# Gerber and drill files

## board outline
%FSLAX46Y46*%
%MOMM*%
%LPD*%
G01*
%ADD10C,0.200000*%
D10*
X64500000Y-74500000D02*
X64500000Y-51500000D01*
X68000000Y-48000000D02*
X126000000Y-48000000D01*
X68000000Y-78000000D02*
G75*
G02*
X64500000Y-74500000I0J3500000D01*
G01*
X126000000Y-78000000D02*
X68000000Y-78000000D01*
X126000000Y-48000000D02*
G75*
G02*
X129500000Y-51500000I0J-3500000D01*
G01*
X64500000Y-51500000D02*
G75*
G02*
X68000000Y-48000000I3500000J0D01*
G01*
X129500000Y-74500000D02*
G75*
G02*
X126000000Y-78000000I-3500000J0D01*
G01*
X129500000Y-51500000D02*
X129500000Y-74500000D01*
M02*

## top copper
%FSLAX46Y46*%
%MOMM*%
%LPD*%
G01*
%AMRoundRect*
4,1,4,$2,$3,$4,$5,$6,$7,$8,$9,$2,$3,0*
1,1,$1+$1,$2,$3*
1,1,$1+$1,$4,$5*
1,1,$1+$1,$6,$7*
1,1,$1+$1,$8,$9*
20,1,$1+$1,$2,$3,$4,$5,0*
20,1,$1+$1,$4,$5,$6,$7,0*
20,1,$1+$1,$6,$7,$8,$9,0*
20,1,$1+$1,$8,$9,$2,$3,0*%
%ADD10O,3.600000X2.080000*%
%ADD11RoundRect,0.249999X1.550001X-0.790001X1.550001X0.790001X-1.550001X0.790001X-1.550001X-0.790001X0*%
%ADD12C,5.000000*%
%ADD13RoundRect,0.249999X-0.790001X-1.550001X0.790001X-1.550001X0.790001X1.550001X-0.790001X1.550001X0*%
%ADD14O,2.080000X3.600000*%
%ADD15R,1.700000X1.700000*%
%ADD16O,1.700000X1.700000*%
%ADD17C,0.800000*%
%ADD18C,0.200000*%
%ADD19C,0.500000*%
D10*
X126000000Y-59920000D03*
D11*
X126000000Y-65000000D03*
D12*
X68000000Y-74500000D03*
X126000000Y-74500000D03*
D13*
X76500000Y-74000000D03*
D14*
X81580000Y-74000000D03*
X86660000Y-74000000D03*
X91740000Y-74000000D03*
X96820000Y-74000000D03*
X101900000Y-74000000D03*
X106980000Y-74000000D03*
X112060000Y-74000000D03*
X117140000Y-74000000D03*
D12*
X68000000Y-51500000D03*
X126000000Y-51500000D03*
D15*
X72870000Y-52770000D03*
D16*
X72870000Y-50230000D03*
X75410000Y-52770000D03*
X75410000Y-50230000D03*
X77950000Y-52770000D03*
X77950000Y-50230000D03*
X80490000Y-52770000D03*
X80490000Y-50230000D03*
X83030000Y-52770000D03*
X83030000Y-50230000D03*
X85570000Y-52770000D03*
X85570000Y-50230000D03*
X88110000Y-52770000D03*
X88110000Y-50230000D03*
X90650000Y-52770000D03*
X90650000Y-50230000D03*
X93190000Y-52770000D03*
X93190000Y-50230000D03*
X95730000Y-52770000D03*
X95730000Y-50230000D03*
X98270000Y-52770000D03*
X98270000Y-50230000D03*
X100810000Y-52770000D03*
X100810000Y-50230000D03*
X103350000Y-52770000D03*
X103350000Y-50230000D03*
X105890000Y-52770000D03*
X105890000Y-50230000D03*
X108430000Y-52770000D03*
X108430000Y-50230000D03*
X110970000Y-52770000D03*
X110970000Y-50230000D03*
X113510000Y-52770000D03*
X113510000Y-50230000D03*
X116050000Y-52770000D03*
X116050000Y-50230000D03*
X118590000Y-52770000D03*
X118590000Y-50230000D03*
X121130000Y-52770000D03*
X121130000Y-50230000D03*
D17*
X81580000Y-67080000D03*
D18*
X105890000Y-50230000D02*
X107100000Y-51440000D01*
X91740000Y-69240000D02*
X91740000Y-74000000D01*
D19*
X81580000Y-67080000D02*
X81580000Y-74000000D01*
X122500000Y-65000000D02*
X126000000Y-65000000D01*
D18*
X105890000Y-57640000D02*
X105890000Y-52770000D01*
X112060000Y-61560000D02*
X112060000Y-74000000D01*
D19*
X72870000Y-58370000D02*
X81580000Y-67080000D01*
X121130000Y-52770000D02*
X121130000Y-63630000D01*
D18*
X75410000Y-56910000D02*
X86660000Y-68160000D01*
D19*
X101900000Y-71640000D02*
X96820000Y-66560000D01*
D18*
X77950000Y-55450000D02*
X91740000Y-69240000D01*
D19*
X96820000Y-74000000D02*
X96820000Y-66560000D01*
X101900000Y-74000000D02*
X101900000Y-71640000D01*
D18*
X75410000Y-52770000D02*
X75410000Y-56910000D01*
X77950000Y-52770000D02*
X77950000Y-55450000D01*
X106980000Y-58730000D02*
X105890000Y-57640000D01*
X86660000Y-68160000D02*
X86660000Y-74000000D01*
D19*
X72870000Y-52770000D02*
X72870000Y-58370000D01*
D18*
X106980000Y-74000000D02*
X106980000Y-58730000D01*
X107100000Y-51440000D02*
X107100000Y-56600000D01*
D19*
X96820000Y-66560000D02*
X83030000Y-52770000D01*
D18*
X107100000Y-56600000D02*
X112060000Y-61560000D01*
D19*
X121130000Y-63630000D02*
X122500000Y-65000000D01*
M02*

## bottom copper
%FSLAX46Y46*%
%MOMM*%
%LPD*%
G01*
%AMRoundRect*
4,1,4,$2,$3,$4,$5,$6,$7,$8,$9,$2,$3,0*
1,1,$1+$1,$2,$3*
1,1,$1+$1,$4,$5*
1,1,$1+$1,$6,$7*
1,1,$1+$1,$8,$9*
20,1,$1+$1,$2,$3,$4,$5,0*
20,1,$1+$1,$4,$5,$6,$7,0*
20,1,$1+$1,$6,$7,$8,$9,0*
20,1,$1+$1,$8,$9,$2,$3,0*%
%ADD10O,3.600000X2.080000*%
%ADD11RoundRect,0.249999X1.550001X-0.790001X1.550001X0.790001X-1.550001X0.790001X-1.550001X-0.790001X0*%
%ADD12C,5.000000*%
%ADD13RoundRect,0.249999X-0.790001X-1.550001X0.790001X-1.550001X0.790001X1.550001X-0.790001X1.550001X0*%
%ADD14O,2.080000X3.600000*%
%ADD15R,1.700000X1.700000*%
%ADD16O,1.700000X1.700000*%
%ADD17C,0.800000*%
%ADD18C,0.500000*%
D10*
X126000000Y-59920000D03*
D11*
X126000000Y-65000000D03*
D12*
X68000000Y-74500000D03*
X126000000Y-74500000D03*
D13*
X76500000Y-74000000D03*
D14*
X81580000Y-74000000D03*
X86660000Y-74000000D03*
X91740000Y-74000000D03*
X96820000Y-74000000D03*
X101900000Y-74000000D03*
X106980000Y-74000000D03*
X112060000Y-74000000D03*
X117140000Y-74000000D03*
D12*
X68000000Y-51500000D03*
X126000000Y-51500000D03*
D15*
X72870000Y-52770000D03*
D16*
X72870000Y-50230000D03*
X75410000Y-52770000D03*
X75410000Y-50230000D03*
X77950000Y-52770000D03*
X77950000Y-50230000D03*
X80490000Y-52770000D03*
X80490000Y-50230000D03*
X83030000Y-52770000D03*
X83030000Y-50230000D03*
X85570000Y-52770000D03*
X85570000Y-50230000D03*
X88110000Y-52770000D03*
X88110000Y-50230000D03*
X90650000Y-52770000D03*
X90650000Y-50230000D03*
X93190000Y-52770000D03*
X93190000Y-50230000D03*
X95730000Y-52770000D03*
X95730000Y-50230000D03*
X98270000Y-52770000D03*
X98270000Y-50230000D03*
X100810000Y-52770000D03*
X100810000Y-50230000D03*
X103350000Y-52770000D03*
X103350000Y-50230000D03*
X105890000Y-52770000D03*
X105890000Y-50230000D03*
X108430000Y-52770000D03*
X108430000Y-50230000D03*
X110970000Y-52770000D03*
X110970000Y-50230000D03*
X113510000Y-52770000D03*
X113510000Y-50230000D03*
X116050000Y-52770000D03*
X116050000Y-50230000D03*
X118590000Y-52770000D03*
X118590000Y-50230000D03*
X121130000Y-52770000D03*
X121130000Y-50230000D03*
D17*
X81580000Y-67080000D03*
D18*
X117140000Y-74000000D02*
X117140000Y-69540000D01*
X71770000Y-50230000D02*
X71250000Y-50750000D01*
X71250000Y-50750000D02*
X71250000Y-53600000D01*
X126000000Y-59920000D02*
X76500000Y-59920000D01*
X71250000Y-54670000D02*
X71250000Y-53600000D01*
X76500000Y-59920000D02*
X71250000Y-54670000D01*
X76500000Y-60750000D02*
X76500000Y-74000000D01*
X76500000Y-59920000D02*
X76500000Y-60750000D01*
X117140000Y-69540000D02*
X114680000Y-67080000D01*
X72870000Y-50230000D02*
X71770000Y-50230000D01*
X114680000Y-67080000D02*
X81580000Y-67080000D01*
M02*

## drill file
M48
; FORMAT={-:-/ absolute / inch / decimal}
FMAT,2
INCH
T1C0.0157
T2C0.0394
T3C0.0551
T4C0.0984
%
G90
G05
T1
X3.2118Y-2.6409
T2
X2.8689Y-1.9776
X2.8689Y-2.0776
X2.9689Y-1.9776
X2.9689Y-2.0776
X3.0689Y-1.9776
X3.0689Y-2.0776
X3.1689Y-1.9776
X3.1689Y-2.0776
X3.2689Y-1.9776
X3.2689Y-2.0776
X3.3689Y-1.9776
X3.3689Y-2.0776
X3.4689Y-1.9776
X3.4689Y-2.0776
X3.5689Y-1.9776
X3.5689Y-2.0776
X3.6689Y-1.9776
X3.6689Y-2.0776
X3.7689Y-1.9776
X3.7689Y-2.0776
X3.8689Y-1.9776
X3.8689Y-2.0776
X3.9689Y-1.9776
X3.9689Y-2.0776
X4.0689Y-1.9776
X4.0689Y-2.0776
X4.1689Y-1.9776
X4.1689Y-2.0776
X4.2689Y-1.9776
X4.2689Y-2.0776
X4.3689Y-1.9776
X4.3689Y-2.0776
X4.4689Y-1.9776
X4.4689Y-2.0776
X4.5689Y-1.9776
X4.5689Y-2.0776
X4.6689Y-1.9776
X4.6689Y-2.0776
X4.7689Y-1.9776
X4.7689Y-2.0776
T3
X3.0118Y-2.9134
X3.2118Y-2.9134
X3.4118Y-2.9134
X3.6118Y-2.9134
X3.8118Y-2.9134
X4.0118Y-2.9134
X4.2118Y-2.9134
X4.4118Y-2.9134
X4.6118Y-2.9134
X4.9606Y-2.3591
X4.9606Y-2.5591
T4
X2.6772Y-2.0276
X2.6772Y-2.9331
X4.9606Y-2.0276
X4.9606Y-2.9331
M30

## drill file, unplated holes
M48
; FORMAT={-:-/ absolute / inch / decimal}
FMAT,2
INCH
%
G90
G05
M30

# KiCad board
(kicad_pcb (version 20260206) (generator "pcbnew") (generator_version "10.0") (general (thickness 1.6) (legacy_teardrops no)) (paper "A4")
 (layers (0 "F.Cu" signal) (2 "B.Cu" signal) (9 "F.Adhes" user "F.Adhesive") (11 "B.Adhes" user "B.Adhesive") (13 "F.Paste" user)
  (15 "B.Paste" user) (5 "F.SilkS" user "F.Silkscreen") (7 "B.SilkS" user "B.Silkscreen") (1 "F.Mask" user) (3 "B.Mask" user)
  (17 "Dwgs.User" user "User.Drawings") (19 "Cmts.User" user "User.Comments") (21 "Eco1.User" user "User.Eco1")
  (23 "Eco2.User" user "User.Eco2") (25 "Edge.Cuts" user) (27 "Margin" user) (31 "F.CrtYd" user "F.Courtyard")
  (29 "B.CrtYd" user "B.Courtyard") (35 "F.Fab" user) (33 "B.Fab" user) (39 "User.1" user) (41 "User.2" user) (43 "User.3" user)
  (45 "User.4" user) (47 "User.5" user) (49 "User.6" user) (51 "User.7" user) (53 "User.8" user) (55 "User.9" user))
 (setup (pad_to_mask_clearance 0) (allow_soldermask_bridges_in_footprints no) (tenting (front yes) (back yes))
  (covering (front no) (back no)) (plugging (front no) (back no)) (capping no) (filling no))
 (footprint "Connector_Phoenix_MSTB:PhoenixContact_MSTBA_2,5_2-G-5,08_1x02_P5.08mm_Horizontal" (layer "F.Cu") (at 126 65 90)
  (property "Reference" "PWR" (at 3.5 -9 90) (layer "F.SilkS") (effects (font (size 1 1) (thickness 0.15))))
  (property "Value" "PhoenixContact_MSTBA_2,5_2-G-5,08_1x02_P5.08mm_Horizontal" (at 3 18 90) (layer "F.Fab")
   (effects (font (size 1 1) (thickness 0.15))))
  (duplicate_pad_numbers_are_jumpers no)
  (pad "1" thru_hole roundrect (at 0 0 90) (size 2.08 3.6) (drill 1.4) (layers "*.Cu" "*.Mask") (remove_unused_layers no)
   (roundrect_rratio 0.120192))
  (pad "2" thru_hole oval (at 5.08 0 90) (size 2.08 3.6) (drill 1.4) (layers "*.Cu" "*.Mask") (remove_unused_layers no)))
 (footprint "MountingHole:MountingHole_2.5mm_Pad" (layer "F.Cu") (at 68 74.5)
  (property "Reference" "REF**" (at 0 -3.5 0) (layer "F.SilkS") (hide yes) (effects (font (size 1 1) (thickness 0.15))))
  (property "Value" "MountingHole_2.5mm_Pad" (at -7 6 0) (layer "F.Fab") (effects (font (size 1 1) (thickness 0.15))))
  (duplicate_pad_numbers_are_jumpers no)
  (pad "1" thru_hole circle (at 0 0) (size 5 5) (drill 2.5) (layers "*.Cu" "*.Mask") (remove_unused_layers no)))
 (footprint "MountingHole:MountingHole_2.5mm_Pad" (layer "F.Cu") (at 126 74.5)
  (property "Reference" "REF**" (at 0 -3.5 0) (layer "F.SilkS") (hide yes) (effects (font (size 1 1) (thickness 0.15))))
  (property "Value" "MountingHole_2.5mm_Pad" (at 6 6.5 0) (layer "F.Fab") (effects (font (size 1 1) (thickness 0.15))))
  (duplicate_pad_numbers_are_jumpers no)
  (pad "1" thru_hole circle (at 0 0) (size 5 5) (drill 2.5) (layers "*.Cu" "*.Mask") (remove_unused_layers no)))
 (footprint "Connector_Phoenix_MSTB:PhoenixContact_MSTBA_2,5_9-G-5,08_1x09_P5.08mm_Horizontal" (layer "F.Cu") (at 76.5 74)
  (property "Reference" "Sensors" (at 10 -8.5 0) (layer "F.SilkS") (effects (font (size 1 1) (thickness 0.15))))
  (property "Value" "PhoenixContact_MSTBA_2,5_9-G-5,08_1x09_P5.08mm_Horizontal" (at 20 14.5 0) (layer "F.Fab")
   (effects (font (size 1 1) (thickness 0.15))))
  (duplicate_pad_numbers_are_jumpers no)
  (pad "1" thru_hole roundrect (at 0 0) (size 2.08 3.6) (drill 1.4) (layers "*.Cu" "*.Mask") (remove_unused_layers no)
   (roundrect_rratio 0.120192))
  (pad "2" thru_hole oval (at 5.08 0) (size 2.08 3.6) (drill 1.4) (layers "*.Cu" "*.Mask") (remove_unused_layers no))
  (pad "3" thru_hole oval (at 10.16 0) (size 2.08 3.6) (drill 1.4) (layers "*.Cu" "*.Mask") (remove_unused_layers no))
  (pad "4" thru_hole oval (at 15.24 0) (size 2.08 3.6) (drill 1.4) (layers "*.Cu" "*.Mask") (remove_unused_layers no))
  (pad "5" thru_hole oval (at 20.32 0) (size 2.08 3.6) (drill 1.4) (layers "*.Cu" "*.Mask") (remove_unused_layers no))
  (pad "6" thru_hole oval (at 25.4 0) (size 2.08 3.6) (drill 1.4) (layers "*.Cu" "*.Mask") (remove_unused_layers no))
  (pad "7" thru_hole oval (at 30.48 0) (size 2.08 3.6) (drill 1.4) (layers "*.Cu" "*.Mask") (remove_unused_layers no))
  (pad "8" thru_hole oval (at 35.56 0) (size 2.08 3.6) (drill 1.4) (layers "*.Cu" "*.Mask") (remove_unused_layers no))
  (pad "9" thru_hole oval (at 40.64 0) (size 2.08 3.6) (drill 1.4) (layers "*.Cu" "*.Mask") (remove_unused_layers no)))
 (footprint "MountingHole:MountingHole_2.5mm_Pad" (layer "F.Cu") (at 68 51.5)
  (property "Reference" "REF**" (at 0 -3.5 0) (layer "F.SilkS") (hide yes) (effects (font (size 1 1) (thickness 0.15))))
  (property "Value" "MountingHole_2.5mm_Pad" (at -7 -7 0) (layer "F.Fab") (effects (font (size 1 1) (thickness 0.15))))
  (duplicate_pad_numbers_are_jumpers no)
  (pad "1" thru_hole circle (at 0 0) (size 5 5) (drill 2.5) (layers "*.Cu" "*.Mask") (remove_unused_layers no)))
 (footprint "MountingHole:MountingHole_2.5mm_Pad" (layer "F.Cu") (at 126 51.5)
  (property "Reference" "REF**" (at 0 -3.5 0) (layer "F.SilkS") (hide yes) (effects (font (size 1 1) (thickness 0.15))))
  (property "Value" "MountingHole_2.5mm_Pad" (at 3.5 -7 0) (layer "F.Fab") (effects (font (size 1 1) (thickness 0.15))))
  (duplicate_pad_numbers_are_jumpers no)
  (pad "1" thru_hole circle (at 0 0) (size 5 5) (drill 2.5) (layers "*.Cu" "*.Mask") (remove_unused_layers no)))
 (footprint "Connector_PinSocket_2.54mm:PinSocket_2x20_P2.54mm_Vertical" (layer "B.Cu") (at 121.16 50.2 90)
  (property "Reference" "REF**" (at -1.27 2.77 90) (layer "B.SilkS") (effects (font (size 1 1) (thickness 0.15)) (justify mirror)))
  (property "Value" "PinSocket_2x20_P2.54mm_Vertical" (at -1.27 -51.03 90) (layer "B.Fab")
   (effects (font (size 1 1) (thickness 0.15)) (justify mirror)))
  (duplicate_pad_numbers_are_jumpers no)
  (pad "1" thru_hole rect (at 0 0 90) (size 1.7 1.7) (drill 1) (layers "*.Cu" "*.Mask") (remove_unused_layers no))
  (pad "2" thru_hole circle (at -2.54 0 90) (size 1.7 1.7) (drill 1) (layers "*.Cu" "*.Mask") (remove_unused_layers no))
  (pad "3" thru_hole circle (at 0 -2.54 90) (size 1.7 1.7) (drill 1) (layers "*.Cu" "*.Mask") (remove_unused_layers no))
  (pad "4" thru_hole circle (at -2.54 -2.54 90) (size 1.7 1.7) (drill 1) (layers "*.Cu" "*.Mask") (remove_unused_layers no))
  (pad "5" thru_hole circle (at 0 -5.08 90) (size 1.7 1.7) (drill 1) (layers "*.Cu" "*.Mask") (remove_unused_layers no))
  (pad "6" thru_hole circle (at -2.54 -5.08 90) (size 1.7 1.7) (drill 1) (layers "*.Cu" "*.Mask") (remove_unused_layers no))
  (pad "7" thru_hole circle (at 0 -7.62 90) (size 1.7 1.7) (drill 1) (layers "*.Cu" "*.Mask") (remove_unused_layers no))
  (pad "8" thru_hole circle (at -2.54 -7.62 90) (size 1.7 1.7) (drill 1) (layers "*.Cu" "*.Mask") (remove_unused_layers no))
  (pad "9" thru_hole circle (at 0 -10.16 90) (size 1.7 1.7) (drill 1) (layers "*.Cu" "*.Mask") (remove_unused_layers no))
  (pad "10" thru_hole circle (at -2.54 -10.16 90) (size 1.7 1.7) (drill 1) (layers "*.Cu" "*.Mask") (remove_unused_layers no))
  (pad "11" thru_hole circle (at 0 -12.7 90) (size 1.7 1.7) (drill 1) (layers "*.Cu" "*.Mask") (remove_unused_layers no))
  (pad "12" thru_hole circle (at -2.54 -12.7 90) (size 1.7 1.7) (drill 1) (layers "*.Cu" "*.Mask") (remove_unused_layers no))
  (pad "13" thru_hole circle (at 0 -15.24 90) (size 1.7 1.7) (drill 1) (layers "*.Cu" "*.Mask") (remove_unused_layers no))
  (pad "14" thru_hole circle (at -2.54 -15.24 90) (size 1.7 1.7) (drill 1) (layers "*.Cu" "*.Mask") (remove_unused_layers no))
  (pad "15" thru_hole circle (at 0 -17.78 90) (size 1.7 1.7) (drill 1) (layers "*.Cu" "*.Mask") (remove_unused_layers no))
  (pad "16" thru_hole circle (at -2.54 -17.78 90) (size 1.7 1.7) (drill 1) (layers "*.Cu" "*.Mask") (remove_unused_layers no))
  (pad "17" thru_hole circle (at 0 -20.32 90) (size 1.7 1.7) (drill 1) (layers "*.Cu" "*.Mask") (remove_unused_layers no))
  (pad "18" thru_hole circle (at -2.54 -20.32 90) (size 1.7 1.7) (drill 1) (layers "*.Cu" "*.Mask") (remove_unused_layers no))
  (pad "19" thru_hole circle (at 0 -22.86 90) (size 1.7 1.7) (drill 1) (layers "*.Cu" "*.Mask") (remove_unused_layers no))
  (pad "20" thru_hole circle (at -2.54 -22.86 90) (size 1.7 1.7) (drill 1) (layers "*.Cu" "*.Mask") (remove_unused_layers no))
  (pad "21" thru_hole circle (at 0 -25.4 90) (size 1.7 1.7) (drill 1) (layers "*.Cu" "*.Mask") (remove_unused_layers no))
  (pad "22" thru_hole circle (at -2.54 -25.4 90) (size 1.7 1.7) (drill 1) (layers "*.Cu" "*.Mask") (remove_unused_layers no))
  (pad "23" thru_hole circle (at 0 -27.94 90) (size 1.7 1.7) (drill 1) (layers "*.Cu" "*.Mask") (remove_unused_layers no))
  (pad "24" thru_hole circle (at -2.54 -27.94 90) (size 1.7 1.7) (drill 1) (layers "*.Cu" "*.Mask") (remove_unused_layers no))
  (pad "25" thru_hole circle (at 0 -30.48 90) (size 1.7 1.7) (drill 1) (layers "*.Cu" "*.Mask") (remove_unused_layers no))
  (pad "26" thru_hole circle (at -2.54 -30.48 90) (size 1.7 1.7) (drill 1) (layers "*.Cu" "*.Mask") (remove_unused_layers no))
  (pad "27" thru_hole circle (at 0 -33.02 90) (size 1.7 1.7) (drill 1) (layers "*.Cu" "*.Mask") (remove_unused_layers no))
  (pad "28" thru_hole circle (at -2.54 -33.02 90) (size 1.7 1.7) (drill 1) (layers "*.Cu" "*.Mask") (remove_unused_layers no))
  (pad "29" thru_hole circle (at 0 -35.56 90) (size 1.7 1.7) (drill 1) (layers "*.Cu" "*.Mask") (remove_unused_layers no))
  (pad "30" thru_hole circle (at -2.54 -35.56 90) (size 1.7 1.7) (drill 1) (layers "*.Cu" "*.Mask") (remove_unused_layers no))
  (pad "31" thru_hole circle (at 0 -38.1 90) (size 1.7 1.7) (drill 1) (layers "*.Cu" "*.Mask") (remove_unused_layers no))
  (pad "32" thru_hole circle (at -2.54 -38.1 90) (size 1.7 1.7) (drill 1) (layers "*.Cu" "*.Mask") (remove_unused_layers no))
  (pad "33" thru_hole circle (at 0 -40.64 90) (size 1.7 1.7) (drill 1) (layers "*.Cu" "*.Mask") (remove_unused_layers no))
  (pad "34" thru_hole circle (at -2.54 -40.64 90) (size 1.7 1.7) (drill 1) (layers "*.Cu" "*.Mask") (remove_unused_layers no))
  (pad "35" thru_hole circle (at 0 -43.18 90) (size 1.7 1.7) (drill 1) (layers "*.Cu" "*.Mask") (remove_unused_layers no))
  (pad "36" thru_hole circle (at -2.54 -43.18 90) (size 1.7 1.7) (drill 1) (layers "*.Cu" "*.Mask") (remove_unused_layers no))
  (pad "37" thru_hole circle (at 0 -45.72 90) (size 1.7 1.7) (drill 1) (layers "*.Cu" "*.Mask") (remove_unused_layers no))
  (pad "38" thru_hole circle (at -2.54 -45.72 90) (size 1.7 1.7) (drill 1) (layers "*.Cu" "*.Mask") (remove_unused_layers no))
  (pad "39" thru_hole circle (at 0 -48.26 90) (size 1.7 1.7) (drill 1) (layers "*.Cu" "*.Mask") (remove_unused_layers no))
  (pad "40" thru_hole circle (at -2.54 -48.26 90) (size 1.7 1.7) (drill 1) (layers "*.Cu" "*.Mask") (remove_unused_layers no)))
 (gr_arc (start 64.5 51.5) (mid 65.525126 49.025126) (end 68 48) (stroke (width 0.2) (type default)) (layer "Edge.Cuts"))
 (gr_line (start 64.5 74.5) (end 64.5 51.5) (stroke (width 0.2) (type default)) (layer "Edge.Cuts"))
 (gr_line (start 68 48) (end 126 48) (stroke (width 0.2) (type default)) (layer "Edge.Cuts"))
 (gr_arc (start 68 78) (mid 65.525126 76.974874) (end 64.5 74.5) (stroke (width 0.2) (type default)) (layer "Edge.Cuts"))
 (gr_arc (start 126 48) (mid 128.474874 49.025126) (end 129.5 51.5) (stroke (width 0.2) (type default)) (layer "Edge.Cuts"))
 (gr_line (start 126 78) (end 68 78) (stroke (width 0.2) (type default)) (layer "Edge.Cuts"))
 (gr_line (start 129.5 51.5) (end 129.5 74.5) (stroke (width 0.2) (type default)) (layer "Edge.Cuts"))
 (gr_arc (start 129.5 74.5) (mid 128.474874 76.974874) (end 126 78) (stroke (width 0.2) (type default)) (layer "Edge.Cuts"))
 (segment (start 105.89 50.23) (end 107.1 51.44) (width 0.2) (layer "F.Cu") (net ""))
 (segment (start 91.74 69.24) (end 91.74 74) (width 0.2) (layer "F.Cu") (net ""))
 (segment (start 81.58 67.08) (end 81.58 74) (width 0.5) (layer "F.Cu") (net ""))
 (segment (start 122.5 65) (end 126 65) (width 0.5) (layer "F.Cu") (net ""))
 (segment (start 105.89 57.64) (end 105.89 52.77) (width 0.2) (layer "F.Cu") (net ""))
 (segment (start 112.06 61.56) (end 112.06 74) (width 0.2) (layer "F.Cu") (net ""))
 (segment (start 72.87 58.37) (end 81.58 67.08) (width 0.5) (layer "F.Cu") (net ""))
 (segment (start 121.13 52.77) (end 121.13 63.63) (width 0.5) (layer "F.Cu") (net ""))
 (segment (start 75.41 56.91) (end 86.66 68.16) (width 0.2) (layer "F.Cu") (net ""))
 (segment (start 101.9 71.64) (end 96.82 66.56) (width 0.5) (layer "F.Cu") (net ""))
 (segment (start 77.95 55.45) (end 91.74 69.24) (width 0.2) (layer "F.Cu") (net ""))
 (segment (start 96.82 74) (end 96.82 66.56) (width 0.5) (layer "F.Cu") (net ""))
 (segment (start 101.9 74) (end 101.9 71.64) (width 0.5) (layer "F.Cu") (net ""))
 (segment (start 75.41 52.77) (end 75.41 56.91) (width 0.2) (layer "F.Cu") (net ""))
 (segment (start 77.95 52.77) (end 77.95 55.45) (width 0.2) (layer "F.Cu") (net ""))
 (segment (start 106.98 58.73) (end 105.89 57.64) (width 0.2) (layer "F.Cu") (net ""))
 (segment (start 86.66 68.16) (end 86.66 74) (width 0.2) (layer "F.Cu") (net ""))
 (segment (start 72.87 52.77) (end 72.87 58.37) (width 0.5) (layer "F.Cu") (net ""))
 (segment (start 106.98 74) (end 106.98 58.73) (width 0.2) (layer "F.Cu") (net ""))
 (segment (start 107.1 51.44) (end 107.1 56.6) (width 0.2) (layer "F.Cu") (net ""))
 (segment (start 96.82 66.56) (end 83.03 52.77) (width 0.5) (layer "F.Cu") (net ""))
 (segment (start 107.1 56.6) (end 112.06 61.56) (width 0.2) (layer "F.Cu") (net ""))
 (segment (start 121.13 63.63) (end 122.5 65) (width 0.5) (layer "F.Cu") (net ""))
 (via (at 81.58 67.08) (size 0.8) (drill 0.4) (layers "F.Cu" "B.Cu") (capping no) (covering (front no) (back no))
  (plugging (front no) (back no)) (filling no) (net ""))
 (segment (start 117.14 74) (end 117.14 69.54) (width 0.5) (layer "B.Cu") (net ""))
 (segment (start 71.77 50.23) (end 71.25 50.75) (width 0.5) (layer "B.Cu") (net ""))
 (segment (start 71.25 50.75) (end 71.25 53.6) (width 0.5) (layer "B.Cu") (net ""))
 (segment (start 126 59.92) (end 76.5 59.92) (width 0.5) (layer "B.Cu") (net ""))
 (segment (start 71.25 54.67) (end 71.25 53.6) (width 0.5) (layer "B.Cu") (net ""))
 (segment (start 76.5 59.92) (end 71.25 54.67) (width 0.5) (layer "B.Cu") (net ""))
 (segment (start 76.5 60.75) (end 76.5 74) (width 0.5) (layer "B.Cu") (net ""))
 (segment (start 76.5 59.92) (end 76.5 60.75) (width 0.5) (layer "B.Cu") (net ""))
 (segment (start 117.14 69.54) (end 114.68 67.08) (width 0.5) (layer "B.Cu") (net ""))
 (segment (start 72.87 50.23) (end 71.77 50.23) (width 0.5) (layer "B.Cu") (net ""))
 (segment (start 114.68 67.08) (end 81.58 67.08) (width 0.5) (layer "B.Cu") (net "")))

